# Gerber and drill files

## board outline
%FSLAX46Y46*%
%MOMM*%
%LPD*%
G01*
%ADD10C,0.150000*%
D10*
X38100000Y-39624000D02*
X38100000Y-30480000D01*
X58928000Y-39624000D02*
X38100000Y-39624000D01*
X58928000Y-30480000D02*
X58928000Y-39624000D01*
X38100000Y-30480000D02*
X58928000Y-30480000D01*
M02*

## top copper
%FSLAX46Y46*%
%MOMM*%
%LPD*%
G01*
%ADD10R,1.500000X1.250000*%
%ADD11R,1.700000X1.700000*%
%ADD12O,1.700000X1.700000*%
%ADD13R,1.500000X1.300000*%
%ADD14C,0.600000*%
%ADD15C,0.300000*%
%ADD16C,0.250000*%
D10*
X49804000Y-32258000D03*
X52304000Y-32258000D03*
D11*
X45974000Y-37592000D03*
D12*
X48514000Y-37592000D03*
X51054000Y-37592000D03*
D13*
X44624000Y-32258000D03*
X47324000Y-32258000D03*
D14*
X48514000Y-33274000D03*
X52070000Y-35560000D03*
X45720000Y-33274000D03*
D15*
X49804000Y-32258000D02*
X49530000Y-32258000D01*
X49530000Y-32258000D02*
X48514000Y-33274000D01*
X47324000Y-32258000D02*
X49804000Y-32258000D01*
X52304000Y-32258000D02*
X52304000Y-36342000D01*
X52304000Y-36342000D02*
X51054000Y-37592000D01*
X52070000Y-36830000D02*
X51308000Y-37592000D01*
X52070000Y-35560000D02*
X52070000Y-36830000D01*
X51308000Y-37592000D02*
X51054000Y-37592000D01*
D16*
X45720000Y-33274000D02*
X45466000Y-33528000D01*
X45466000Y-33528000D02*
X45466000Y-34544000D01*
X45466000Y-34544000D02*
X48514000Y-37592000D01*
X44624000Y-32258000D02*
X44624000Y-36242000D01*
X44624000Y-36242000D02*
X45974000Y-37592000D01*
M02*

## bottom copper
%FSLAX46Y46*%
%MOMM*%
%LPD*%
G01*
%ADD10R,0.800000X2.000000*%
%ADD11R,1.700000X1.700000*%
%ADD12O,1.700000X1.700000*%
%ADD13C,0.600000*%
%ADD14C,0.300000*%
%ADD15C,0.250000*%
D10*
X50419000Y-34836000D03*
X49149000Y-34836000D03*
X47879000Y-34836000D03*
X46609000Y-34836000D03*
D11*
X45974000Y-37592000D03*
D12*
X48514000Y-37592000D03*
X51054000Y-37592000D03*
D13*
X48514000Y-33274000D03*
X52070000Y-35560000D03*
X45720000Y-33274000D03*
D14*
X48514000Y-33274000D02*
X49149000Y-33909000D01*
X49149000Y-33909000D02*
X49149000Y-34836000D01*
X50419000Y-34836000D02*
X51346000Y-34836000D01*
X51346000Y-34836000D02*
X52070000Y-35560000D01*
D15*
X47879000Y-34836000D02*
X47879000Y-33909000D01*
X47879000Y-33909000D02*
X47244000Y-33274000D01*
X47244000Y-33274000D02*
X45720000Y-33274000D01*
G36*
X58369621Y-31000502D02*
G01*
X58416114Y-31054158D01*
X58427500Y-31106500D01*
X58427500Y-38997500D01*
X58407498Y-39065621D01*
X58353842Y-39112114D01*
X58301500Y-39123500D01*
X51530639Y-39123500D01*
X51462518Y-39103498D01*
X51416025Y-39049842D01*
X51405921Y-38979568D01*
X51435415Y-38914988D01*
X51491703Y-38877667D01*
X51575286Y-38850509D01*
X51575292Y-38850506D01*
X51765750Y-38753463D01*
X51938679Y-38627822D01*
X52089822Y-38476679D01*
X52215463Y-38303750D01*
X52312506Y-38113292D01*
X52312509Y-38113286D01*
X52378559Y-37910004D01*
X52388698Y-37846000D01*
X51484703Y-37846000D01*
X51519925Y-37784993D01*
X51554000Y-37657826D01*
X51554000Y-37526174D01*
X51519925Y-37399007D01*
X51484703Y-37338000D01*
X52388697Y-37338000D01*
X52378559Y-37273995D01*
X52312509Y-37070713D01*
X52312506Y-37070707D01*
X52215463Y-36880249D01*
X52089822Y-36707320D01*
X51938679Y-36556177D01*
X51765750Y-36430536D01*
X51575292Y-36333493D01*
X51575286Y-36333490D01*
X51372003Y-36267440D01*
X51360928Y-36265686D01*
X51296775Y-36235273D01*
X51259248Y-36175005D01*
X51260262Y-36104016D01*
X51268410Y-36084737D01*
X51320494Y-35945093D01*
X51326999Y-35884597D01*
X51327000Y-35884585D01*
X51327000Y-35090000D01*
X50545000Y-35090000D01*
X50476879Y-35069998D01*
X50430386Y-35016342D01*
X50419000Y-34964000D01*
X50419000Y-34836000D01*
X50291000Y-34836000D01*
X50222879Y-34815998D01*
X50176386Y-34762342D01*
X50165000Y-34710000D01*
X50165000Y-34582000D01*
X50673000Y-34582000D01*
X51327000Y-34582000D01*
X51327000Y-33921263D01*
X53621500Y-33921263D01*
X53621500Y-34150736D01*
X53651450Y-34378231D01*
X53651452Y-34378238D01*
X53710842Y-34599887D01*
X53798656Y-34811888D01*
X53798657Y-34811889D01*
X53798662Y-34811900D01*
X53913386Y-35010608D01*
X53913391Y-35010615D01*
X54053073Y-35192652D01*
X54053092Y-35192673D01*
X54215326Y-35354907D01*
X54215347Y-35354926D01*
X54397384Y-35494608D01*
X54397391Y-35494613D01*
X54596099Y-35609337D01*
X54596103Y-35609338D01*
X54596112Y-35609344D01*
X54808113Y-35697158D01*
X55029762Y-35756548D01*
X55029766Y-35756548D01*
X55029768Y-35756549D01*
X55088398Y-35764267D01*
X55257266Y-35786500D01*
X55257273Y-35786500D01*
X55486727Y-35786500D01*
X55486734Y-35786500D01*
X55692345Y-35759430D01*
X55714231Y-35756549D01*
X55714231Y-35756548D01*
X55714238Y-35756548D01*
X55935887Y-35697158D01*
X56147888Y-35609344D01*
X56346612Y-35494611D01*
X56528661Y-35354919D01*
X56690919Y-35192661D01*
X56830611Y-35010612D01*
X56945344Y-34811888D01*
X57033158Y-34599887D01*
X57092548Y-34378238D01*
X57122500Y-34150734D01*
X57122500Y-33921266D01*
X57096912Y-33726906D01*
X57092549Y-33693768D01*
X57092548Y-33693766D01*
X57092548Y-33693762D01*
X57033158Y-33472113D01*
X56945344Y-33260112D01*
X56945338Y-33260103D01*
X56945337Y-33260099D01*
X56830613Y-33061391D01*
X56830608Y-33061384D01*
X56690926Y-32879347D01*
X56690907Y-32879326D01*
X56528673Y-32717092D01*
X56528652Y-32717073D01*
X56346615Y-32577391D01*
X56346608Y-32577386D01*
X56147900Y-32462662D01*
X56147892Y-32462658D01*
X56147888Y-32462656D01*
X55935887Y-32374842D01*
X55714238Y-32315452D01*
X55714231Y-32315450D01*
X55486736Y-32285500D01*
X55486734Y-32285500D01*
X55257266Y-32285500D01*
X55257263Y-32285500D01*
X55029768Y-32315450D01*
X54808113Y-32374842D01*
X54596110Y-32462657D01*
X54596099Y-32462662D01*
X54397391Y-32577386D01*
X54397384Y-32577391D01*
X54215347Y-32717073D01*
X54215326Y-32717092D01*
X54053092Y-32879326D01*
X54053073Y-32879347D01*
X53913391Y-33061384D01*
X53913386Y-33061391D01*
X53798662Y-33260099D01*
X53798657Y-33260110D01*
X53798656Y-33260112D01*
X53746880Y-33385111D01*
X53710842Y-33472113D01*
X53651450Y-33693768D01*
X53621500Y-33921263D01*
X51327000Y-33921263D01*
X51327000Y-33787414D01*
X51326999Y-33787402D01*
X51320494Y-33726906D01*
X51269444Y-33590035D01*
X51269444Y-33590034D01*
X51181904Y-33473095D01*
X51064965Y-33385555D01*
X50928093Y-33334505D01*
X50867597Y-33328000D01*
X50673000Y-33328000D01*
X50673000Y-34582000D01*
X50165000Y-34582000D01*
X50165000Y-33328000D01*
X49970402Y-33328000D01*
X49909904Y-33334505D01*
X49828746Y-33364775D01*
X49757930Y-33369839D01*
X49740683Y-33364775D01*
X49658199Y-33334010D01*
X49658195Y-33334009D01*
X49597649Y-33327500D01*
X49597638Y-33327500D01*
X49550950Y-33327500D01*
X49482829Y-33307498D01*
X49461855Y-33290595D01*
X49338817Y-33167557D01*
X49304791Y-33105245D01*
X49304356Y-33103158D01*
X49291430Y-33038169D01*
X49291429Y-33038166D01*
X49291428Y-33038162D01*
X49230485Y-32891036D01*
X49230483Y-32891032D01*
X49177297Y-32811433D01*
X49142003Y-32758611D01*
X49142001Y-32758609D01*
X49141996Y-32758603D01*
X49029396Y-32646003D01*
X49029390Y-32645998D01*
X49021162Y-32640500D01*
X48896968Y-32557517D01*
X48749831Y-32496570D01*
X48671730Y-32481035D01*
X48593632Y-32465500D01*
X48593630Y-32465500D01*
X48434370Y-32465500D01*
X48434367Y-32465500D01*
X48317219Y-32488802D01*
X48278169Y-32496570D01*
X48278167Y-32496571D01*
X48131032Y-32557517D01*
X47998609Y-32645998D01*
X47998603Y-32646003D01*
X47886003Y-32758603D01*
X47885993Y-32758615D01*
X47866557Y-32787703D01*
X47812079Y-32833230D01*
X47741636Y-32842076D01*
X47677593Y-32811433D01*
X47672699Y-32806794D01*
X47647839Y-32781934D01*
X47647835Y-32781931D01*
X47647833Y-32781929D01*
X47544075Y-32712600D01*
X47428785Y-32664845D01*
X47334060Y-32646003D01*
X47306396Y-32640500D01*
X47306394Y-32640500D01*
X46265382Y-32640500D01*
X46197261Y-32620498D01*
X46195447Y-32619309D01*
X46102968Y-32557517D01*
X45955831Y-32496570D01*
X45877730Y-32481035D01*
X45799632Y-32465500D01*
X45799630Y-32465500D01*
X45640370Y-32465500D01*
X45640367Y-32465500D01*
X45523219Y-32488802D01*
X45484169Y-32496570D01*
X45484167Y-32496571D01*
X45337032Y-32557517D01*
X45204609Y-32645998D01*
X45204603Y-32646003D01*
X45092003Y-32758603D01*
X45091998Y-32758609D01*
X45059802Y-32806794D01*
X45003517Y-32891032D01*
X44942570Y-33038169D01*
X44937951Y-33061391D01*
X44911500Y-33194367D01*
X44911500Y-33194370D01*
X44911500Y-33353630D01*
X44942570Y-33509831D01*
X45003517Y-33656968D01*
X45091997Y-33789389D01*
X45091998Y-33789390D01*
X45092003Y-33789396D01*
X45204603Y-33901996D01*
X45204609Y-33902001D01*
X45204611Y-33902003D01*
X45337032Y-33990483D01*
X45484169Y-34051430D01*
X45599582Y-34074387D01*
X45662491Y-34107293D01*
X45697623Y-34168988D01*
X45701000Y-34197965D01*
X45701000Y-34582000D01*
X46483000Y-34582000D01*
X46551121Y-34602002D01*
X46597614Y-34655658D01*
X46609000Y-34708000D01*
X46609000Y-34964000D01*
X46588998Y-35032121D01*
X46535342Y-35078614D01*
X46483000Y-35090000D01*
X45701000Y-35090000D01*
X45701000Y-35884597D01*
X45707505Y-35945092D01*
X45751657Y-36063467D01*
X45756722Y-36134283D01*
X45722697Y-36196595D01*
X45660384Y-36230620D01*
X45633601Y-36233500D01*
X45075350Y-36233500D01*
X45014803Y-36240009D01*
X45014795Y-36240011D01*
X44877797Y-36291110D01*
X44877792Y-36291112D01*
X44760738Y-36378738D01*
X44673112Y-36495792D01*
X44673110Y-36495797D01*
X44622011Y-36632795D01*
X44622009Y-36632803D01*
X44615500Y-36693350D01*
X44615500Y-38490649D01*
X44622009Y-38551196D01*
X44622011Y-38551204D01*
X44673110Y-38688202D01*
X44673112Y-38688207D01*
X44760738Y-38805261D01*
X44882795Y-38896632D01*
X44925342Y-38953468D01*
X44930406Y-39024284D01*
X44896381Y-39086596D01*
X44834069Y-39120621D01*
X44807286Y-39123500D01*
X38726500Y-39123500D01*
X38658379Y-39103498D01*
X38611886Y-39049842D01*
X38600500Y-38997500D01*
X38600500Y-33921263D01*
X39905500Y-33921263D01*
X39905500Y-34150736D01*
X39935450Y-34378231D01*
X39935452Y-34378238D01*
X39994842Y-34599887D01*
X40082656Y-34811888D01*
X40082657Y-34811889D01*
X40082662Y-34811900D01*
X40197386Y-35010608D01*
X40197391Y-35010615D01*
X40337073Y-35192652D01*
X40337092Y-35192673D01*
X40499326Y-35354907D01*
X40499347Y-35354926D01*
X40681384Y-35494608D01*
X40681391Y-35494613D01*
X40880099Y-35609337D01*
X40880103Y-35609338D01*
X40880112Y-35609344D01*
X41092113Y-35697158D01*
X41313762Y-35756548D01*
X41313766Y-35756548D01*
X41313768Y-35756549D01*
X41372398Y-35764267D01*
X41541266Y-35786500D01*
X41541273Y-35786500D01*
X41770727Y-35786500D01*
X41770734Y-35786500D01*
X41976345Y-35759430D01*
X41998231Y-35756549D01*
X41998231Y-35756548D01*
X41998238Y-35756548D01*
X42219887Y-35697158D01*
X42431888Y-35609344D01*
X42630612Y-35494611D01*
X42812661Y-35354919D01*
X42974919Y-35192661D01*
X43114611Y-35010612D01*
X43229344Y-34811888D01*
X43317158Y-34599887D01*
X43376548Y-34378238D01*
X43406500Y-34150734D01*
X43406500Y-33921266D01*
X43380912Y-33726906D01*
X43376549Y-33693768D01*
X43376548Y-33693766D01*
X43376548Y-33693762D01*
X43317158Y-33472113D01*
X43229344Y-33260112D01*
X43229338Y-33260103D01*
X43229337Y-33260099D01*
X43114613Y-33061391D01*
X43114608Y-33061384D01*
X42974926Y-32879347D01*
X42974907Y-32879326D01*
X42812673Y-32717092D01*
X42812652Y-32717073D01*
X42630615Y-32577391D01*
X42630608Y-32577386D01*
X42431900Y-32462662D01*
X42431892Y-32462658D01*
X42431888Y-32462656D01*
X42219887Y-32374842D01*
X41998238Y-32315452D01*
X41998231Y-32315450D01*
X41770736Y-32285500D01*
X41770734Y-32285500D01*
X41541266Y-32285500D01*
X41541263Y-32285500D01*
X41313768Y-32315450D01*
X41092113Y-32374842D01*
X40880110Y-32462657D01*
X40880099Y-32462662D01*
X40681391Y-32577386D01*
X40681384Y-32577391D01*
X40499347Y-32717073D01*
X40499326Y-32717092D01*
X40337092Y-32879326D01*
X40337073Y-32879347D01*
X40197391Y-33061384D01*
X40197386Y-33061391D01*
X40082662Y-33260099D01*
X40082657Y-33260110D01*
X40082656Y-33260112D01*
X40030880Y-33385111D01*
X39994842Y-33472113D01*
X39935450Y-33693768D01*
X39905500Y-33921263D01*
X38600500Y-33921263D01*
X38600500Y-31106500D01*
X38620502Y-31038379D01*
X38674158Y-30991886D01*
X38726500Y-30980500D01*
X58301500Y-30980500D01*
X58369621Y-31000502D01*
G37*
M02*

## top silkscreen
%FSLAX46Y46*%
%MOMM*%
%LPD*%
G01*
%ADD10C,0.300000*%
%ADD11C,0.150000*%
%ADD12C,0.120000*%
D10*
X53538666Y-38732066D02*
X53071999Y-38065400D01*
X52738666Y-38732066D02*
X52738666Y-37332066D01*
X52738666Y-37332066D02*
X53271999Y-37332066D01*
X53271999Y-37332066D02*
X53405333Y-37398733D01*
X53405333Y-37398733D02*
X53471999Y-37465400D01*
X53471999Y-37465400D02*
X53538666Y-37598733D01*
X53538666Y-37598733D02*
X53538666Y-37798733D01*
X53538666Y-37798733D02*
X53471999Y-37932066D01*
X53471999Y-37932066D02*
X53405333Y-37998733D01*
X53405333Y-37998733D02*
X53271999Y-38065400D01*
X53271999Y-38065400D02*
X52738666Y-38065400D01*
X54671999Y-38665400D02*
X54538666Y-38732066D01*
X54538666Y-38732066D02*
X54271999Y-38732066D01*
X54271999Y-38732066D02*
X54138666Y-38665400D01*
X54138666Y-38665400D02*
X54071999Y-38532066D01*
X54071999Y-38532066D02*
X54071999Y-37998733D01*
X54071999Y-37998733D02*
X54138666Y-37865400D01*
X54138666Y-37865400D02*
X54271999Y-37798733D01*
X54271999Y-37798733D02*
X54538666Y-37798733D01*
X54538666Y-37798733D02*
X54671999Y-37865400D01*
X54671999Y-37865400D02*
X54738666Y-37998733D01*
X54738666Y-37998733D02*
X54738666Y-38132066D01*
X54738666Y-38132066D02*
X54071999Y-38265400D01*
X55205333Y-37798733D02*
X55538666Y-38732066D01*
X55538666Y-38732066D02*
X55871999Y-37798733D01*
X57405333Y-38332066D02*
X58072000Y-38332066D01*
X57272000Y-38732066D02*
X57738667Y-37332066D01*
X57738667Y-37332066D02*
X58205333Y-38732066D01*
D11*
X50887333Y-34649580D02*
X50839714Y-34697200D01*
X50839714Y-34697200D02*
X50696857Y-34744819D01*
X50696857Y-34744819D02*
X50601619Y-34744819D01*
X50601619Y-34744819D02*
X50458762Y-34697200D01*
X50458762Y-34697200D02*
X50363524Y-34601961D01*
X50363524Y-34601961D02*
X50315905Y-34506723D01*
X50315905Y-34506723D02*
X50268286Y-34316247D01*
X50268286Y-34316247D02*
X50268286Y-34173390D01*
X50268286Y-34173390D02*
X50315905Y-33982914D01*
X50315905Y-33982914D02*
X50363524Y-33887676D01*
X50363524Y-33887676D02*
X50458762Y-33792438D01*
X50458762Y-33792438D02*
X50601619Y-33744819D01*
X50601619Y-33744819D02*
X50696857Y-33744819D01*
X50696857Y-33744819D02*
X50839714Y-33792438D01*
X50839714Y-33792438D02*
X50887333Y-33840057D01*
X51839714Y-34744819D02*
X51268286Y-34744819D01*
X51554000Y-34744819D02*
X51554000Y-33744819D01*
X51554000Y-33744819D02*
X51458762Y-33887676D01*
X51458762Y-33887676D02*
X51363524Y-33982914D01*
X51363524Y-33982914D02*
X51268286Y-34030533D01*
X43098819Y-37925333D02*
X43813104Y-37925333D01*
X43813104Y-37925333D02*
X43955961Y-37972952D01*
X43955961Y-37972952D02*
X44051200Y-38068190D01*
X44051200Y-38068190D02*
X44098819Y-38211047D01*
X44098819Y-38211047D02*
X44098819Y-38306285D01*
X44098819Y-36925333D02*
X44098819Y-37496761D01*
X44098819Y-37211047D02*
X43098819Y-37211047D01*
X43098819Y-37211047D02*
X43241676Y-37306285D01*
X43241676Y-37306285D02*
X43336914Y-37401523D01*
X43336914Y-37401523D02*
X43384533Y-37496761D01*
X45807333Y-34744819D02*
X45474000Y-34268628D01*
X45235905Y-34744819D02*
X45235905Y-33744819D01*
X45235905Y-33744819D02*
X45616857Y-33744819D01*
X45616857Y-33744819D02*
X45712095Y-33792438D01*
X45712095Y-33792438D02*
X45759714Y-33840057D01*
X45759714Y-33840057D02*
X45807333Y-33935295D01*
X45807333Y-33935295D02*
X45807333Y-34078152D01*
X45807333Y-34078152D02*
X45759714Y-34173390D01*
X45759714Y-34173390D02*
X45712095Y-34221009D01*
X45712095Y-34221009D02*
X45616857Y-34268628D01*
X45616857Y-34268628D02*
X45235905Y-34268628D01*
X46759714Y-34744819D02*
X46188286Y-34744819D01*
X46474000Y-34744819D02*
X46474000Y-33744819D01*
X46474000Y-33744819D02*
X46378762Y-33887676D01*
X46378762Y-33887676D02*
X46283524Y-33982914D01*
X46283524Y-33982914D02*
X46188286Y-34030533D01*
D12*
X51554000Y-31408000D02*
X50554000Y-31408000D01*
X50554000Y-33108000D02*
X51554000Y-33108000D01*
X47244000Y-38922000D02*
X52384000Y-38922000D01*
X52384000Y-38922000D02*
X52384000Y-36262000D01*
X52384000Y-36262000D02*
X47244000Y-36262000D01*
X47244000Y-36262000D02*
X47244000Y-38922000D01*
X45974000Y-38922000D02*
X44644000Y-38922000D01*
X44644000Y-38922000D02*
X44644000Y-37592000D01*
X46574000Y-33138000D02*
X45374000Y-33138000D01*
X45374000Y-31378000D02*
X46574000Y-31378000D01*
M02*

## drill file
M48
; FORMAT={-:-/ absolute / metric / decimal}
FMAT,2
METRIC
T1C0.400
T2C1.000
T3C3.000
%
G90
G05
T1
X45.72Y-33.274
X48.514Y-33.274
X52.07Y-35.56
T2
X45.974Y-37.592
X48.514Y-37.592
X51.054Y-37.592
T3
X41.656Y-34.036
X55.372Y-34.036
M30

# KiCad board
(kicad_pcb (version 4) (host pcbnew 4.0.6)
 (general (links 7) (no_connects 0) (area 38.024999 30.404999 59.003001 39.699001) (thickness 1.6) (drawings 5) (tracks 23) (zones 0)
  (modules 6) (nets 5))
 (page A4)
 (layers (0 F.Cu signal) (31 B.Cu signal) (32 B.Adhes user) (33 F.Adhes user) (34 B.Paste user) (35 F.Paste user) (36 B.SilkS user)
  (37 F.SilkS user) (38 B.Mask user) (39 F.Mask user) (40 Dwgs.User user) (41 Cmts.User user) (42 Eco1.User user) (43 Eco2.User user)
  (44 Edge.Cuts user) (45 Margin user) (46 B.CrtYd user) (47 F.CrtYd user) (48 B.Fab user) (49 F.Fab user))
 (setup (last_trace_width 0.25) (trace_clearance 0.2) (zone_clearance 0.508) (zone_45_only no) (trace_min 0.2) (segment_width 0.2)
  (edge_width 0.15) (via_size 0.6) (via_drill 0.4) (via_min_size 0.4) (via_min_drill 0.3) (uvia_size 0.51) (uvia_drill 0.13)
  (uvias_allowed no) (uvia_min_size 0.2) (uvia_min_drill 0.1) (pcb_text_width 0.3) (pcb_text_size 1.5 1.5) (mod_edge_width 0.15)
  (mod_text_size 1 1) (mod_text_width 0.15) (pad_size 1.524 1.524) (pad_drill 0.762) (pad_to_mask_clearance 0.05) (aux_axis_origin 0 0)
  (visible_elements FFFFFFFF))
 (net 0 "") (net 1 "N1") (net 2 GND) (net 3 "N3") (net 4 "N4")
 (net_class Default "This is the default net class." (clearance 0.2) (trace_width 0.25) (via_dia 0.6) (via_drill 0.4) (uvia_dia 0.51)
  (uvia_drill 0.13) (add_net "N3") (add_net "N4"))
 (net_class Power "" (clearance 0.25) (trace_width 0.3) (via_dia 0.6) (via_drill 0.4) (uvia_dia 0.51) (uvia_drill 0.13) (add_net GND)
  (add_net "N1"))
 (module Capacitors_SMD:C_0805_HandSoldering (layer F.Cu) (at 51.054 32.258)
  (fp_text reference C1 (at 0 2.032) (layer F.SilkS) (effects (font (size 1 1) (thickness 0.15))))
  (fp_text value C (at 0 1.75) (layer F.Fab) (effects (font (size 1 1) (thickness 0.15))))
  (fp_line (start 0.5 -0.85) (end -0.5 -0.85) (layer F.SilkS) (width 0.12))
  (fp_line (start -0.5 0.85) (end 0.5 0.85) (layer F.SilkS) (width 0.12))
  (pad 1 smd rect (at -1.25 0) (size 1.5 1.25) (layers F.Cu F.Paste F.Mask) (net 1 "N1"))
  (pad 2 smd rect (at 1.25 0) (size 1.5 1.25) (layers F.Cu F.Paste F.Mask) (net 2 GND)))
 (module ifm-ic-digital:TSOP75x (layer B.Cu) (at 48.514 34.036 180)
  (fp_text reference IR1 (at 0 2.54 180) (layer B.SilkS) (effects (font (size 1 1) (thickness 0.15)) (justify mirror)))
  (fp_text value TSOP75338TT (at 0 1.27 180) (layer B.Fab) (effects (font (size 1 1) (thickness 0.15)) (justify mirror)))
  (pad 1 smd rect (at -1.905 -0.8 180) (size 0.8 2) (layers B.Cu B.Paste B.Mask) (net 2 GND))
  (pad 2 smd rect (at -0.635 -0.8 180) (size 0.8 2) (layers B.Cu B.Paste B.Mask) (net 1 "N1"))
  (pad 3 smd rect (at 0.635 -0.8 180) (size 0.8 2) (layers B.Cu B.Paste B.Mask) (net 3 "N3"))
  (pad 4 smd rect (at 1.905 -0.8 180) (size 0.8 2) (layers B.Cu B.Paste B.Mask) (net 2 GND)))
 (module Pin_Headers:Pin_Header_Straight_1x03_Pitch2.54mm (layer F.Cu) (at 45.974 37.592 90)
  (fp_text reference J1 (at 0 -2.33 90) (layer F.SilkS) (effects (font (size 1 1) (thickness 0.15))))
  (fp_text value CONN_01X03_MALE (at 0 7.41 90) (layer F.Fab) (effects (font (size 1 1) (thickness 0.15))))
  (fp_line (start -1.33 1.27) (end -1.33 6.41) (layer F.SilkS) (width 0.12))
  (fp_line (start -1.33 6.41) (end 1.33 6.41) (layer F.SilkS) (width 0.12))
  (fp_line (start 1.33 6.41) (end 1.33 1.27) (layer F.SilkS) (width 0.12))
  (fp_line (start 1.33 1.27) (end -1.33 1.27) (layer F.SilkS) (width 0.12))
  (fp_line (start -1.33 0) (end -1.33 -1.33) (layer F.SilkS) (width 0.12))
  (fp_line (start -1.33 -1.33) (end 0 -1.33) (layer F.SilkS) (width 0.12))
  (pad 1 thru_hole rect (at 0 0 90) (size 1.7 1.7) (drill 1) (layers *.Cu *.Mask) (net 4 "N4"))
  (pad 2 thru_hole oval (at 0 2.54 90) (size 1.7 1.7) (drill 1) (layers *.Cu *.Mask) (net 3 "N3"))
  (pad 3 thru_hole oval (at 0 5.08 90) (size 1.7 1.7) (drill 1) (layers *.Cu *.Mask) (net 2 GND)))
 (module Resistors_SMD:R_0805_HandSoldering (layer F.Cu) (at 45.974 32.258)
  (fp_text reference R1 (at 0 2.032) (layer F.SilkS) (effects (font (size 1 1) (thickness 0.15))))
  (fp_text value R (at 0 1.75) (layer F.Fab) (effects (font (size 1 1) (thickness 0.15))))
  (fp_line (start 0.6 0.88) (end -0.6 0.88) (layer F.SilkS) (width 0.12))
  (fp_line (start -0.6 -0.88) (end 0.6 -0.88) (layer F.SilkS) (width 0.12))
  (pad 1 smd rect (at -1.35 0) (size 1.5 1.3) (layers F.Cu F.Paste F.Mask) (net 4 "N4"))
  (pad 2 smd rect (at 1.35 0) (size 1.5 1.3) (layers F.Cu F.Paste F.Mask) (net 1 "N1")))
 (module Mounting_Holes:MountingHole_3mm (layer F.Cu) (at 55.372 34.036)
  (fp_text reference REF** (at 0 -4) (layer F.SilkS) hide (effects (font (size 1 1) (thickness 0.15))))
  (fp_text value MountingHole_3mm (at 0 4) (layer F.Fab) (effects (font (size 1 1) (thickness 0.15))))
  (pad 1 np_thru_hole circle (at 0 0) (size 3 3) (drill 3) (layers *.Cu *.Mask)))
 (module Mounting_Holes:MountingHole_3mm (layer F.Cu) (at 41.656 34.036)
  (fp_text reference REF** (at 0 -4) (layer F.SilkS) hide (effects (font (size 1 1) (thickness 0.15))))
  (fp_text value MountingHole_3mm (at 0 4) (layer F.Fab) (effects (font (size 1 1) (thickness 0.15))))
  (pad 1 np_thru_hole circle (at 0 0) (size 3 3) (drill 3) (layers *.Cu *.Mask)))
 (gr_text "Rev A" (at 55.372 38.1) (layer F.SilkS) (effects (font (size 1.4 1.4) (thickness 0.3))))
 (gr_line (start 38.1 39.624) (end 38.1 30.48) (angle 90) (layer Edge.Cuts) (width 0.15))
 (gr_line (start 58.928 39.624) (end 38.1 39.624) (angle 90) (layer Edge.Cuts) (width 0.15))
 (gr_line (start 58.928 30.48) (end 58.928 39.624) (angle 90) (layer Edge.Cuts) (width 0.15))
 (gr_line (start 38.1 30.48) (end 58.928 30.48) (angle 90) (layer Edge.Cuts) (width 0.15))
 (segment (start 49.804 32.258) (end 49.53 32.258) (width 0.3) (layer F.Cu) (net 1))
 (segment (start 49.53 32.258) (end 48.514 33.274) (width 0.3) (layer F.Cu) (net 1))
 (segment (start 48.514 33.274) (end 49.149 33.909) (width 0.3) (layer B.Cu) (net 1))
 (via (at 48.514 33.274) (size 0.6) (drill 0.4) (layers F.Cu B.Cu) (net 1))
 (segment (start 49.149 33.909) (end 49.149 34.836) (width 0.3) (layer B.Cu) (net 1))
 (segment (start 47.324 32.258) (end 49.804 32.258) (width 0.3) (layer F.Cu) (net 1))
 (segment (start 52.304 32.258) (end 52.304 36.342) (width 0.3) (layer F.Cu) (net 2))
 (segment (start 52.304 36.342) (end 51.054 37.592) (width 0.3) (layer F.Cu) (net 2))
 (segment (start 50.419 34.836) (end 51.346 34.836) (width 0.3) (layer B.Cu) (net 2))
 (segment (start 52.07 36.83) (end 51.308 37.592) (width 0.3) (layer F.Cu) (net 2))
 (segment (start 52.07 35.56) (end 52.07 36.83) (width 0.3) (layer F.Cu) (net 2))
 (via (at 52.07 35.56) (size 0.6) (drill 0.4) (layers F.Cu B.Cu) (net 2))
 (segment (start 51.346 34.836) (end 52.07 35.56) (width 0.3) (layer B.Cu) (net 2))
 (segment (start 51.308 37.592) (end 51.054 37.592) (width 0.3) (layer F.Cu) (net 2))
 (segment (start 47.879 34.836) (end 47.879 33.909) (width 0.25) (layer B.Cu) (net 3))
 (segment (start 47.879 33.909) (end 47.244 33.274) (width 0.25) (layer B.Cu) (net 3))
 (segment (start 47.244 33.274) (end 45.72 33.274) (width 0.25) (layer B.Cu) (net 3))
 (via (at 45.72 33.274) (size 0.6) (drill 0.4) (layers F.Cu B.Cu) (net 3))
 (segment (start 45.72 33.274) (end 45.466 33.528) (width 0.25) (layer F.Cu) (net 3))
 (segment (start 45.466 33.528) (end 45.466 34.544) (width 0.25) (layer F.Cu) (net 3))
 (segment (start 45.466 34.544) (end 48.514 37.592) (width 0.25) (layer F.Cu) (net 3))
 (segment (start 44.624 32.258) (end 44.624 36.242) (width 0.25) (layer F.Cu) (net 4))
 (segment (start 44.624 36.242) (end 45.974 37.592) (width 0.25) (layer F.Cu) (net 4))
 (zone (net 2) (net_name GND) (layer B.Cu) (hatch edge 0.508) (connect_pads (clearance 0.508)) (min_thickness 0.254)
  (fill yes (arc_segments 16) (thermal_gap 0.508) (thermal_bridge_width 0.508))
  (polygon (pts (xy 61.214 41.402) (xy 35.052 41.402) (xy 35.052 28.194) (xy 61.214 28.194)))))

